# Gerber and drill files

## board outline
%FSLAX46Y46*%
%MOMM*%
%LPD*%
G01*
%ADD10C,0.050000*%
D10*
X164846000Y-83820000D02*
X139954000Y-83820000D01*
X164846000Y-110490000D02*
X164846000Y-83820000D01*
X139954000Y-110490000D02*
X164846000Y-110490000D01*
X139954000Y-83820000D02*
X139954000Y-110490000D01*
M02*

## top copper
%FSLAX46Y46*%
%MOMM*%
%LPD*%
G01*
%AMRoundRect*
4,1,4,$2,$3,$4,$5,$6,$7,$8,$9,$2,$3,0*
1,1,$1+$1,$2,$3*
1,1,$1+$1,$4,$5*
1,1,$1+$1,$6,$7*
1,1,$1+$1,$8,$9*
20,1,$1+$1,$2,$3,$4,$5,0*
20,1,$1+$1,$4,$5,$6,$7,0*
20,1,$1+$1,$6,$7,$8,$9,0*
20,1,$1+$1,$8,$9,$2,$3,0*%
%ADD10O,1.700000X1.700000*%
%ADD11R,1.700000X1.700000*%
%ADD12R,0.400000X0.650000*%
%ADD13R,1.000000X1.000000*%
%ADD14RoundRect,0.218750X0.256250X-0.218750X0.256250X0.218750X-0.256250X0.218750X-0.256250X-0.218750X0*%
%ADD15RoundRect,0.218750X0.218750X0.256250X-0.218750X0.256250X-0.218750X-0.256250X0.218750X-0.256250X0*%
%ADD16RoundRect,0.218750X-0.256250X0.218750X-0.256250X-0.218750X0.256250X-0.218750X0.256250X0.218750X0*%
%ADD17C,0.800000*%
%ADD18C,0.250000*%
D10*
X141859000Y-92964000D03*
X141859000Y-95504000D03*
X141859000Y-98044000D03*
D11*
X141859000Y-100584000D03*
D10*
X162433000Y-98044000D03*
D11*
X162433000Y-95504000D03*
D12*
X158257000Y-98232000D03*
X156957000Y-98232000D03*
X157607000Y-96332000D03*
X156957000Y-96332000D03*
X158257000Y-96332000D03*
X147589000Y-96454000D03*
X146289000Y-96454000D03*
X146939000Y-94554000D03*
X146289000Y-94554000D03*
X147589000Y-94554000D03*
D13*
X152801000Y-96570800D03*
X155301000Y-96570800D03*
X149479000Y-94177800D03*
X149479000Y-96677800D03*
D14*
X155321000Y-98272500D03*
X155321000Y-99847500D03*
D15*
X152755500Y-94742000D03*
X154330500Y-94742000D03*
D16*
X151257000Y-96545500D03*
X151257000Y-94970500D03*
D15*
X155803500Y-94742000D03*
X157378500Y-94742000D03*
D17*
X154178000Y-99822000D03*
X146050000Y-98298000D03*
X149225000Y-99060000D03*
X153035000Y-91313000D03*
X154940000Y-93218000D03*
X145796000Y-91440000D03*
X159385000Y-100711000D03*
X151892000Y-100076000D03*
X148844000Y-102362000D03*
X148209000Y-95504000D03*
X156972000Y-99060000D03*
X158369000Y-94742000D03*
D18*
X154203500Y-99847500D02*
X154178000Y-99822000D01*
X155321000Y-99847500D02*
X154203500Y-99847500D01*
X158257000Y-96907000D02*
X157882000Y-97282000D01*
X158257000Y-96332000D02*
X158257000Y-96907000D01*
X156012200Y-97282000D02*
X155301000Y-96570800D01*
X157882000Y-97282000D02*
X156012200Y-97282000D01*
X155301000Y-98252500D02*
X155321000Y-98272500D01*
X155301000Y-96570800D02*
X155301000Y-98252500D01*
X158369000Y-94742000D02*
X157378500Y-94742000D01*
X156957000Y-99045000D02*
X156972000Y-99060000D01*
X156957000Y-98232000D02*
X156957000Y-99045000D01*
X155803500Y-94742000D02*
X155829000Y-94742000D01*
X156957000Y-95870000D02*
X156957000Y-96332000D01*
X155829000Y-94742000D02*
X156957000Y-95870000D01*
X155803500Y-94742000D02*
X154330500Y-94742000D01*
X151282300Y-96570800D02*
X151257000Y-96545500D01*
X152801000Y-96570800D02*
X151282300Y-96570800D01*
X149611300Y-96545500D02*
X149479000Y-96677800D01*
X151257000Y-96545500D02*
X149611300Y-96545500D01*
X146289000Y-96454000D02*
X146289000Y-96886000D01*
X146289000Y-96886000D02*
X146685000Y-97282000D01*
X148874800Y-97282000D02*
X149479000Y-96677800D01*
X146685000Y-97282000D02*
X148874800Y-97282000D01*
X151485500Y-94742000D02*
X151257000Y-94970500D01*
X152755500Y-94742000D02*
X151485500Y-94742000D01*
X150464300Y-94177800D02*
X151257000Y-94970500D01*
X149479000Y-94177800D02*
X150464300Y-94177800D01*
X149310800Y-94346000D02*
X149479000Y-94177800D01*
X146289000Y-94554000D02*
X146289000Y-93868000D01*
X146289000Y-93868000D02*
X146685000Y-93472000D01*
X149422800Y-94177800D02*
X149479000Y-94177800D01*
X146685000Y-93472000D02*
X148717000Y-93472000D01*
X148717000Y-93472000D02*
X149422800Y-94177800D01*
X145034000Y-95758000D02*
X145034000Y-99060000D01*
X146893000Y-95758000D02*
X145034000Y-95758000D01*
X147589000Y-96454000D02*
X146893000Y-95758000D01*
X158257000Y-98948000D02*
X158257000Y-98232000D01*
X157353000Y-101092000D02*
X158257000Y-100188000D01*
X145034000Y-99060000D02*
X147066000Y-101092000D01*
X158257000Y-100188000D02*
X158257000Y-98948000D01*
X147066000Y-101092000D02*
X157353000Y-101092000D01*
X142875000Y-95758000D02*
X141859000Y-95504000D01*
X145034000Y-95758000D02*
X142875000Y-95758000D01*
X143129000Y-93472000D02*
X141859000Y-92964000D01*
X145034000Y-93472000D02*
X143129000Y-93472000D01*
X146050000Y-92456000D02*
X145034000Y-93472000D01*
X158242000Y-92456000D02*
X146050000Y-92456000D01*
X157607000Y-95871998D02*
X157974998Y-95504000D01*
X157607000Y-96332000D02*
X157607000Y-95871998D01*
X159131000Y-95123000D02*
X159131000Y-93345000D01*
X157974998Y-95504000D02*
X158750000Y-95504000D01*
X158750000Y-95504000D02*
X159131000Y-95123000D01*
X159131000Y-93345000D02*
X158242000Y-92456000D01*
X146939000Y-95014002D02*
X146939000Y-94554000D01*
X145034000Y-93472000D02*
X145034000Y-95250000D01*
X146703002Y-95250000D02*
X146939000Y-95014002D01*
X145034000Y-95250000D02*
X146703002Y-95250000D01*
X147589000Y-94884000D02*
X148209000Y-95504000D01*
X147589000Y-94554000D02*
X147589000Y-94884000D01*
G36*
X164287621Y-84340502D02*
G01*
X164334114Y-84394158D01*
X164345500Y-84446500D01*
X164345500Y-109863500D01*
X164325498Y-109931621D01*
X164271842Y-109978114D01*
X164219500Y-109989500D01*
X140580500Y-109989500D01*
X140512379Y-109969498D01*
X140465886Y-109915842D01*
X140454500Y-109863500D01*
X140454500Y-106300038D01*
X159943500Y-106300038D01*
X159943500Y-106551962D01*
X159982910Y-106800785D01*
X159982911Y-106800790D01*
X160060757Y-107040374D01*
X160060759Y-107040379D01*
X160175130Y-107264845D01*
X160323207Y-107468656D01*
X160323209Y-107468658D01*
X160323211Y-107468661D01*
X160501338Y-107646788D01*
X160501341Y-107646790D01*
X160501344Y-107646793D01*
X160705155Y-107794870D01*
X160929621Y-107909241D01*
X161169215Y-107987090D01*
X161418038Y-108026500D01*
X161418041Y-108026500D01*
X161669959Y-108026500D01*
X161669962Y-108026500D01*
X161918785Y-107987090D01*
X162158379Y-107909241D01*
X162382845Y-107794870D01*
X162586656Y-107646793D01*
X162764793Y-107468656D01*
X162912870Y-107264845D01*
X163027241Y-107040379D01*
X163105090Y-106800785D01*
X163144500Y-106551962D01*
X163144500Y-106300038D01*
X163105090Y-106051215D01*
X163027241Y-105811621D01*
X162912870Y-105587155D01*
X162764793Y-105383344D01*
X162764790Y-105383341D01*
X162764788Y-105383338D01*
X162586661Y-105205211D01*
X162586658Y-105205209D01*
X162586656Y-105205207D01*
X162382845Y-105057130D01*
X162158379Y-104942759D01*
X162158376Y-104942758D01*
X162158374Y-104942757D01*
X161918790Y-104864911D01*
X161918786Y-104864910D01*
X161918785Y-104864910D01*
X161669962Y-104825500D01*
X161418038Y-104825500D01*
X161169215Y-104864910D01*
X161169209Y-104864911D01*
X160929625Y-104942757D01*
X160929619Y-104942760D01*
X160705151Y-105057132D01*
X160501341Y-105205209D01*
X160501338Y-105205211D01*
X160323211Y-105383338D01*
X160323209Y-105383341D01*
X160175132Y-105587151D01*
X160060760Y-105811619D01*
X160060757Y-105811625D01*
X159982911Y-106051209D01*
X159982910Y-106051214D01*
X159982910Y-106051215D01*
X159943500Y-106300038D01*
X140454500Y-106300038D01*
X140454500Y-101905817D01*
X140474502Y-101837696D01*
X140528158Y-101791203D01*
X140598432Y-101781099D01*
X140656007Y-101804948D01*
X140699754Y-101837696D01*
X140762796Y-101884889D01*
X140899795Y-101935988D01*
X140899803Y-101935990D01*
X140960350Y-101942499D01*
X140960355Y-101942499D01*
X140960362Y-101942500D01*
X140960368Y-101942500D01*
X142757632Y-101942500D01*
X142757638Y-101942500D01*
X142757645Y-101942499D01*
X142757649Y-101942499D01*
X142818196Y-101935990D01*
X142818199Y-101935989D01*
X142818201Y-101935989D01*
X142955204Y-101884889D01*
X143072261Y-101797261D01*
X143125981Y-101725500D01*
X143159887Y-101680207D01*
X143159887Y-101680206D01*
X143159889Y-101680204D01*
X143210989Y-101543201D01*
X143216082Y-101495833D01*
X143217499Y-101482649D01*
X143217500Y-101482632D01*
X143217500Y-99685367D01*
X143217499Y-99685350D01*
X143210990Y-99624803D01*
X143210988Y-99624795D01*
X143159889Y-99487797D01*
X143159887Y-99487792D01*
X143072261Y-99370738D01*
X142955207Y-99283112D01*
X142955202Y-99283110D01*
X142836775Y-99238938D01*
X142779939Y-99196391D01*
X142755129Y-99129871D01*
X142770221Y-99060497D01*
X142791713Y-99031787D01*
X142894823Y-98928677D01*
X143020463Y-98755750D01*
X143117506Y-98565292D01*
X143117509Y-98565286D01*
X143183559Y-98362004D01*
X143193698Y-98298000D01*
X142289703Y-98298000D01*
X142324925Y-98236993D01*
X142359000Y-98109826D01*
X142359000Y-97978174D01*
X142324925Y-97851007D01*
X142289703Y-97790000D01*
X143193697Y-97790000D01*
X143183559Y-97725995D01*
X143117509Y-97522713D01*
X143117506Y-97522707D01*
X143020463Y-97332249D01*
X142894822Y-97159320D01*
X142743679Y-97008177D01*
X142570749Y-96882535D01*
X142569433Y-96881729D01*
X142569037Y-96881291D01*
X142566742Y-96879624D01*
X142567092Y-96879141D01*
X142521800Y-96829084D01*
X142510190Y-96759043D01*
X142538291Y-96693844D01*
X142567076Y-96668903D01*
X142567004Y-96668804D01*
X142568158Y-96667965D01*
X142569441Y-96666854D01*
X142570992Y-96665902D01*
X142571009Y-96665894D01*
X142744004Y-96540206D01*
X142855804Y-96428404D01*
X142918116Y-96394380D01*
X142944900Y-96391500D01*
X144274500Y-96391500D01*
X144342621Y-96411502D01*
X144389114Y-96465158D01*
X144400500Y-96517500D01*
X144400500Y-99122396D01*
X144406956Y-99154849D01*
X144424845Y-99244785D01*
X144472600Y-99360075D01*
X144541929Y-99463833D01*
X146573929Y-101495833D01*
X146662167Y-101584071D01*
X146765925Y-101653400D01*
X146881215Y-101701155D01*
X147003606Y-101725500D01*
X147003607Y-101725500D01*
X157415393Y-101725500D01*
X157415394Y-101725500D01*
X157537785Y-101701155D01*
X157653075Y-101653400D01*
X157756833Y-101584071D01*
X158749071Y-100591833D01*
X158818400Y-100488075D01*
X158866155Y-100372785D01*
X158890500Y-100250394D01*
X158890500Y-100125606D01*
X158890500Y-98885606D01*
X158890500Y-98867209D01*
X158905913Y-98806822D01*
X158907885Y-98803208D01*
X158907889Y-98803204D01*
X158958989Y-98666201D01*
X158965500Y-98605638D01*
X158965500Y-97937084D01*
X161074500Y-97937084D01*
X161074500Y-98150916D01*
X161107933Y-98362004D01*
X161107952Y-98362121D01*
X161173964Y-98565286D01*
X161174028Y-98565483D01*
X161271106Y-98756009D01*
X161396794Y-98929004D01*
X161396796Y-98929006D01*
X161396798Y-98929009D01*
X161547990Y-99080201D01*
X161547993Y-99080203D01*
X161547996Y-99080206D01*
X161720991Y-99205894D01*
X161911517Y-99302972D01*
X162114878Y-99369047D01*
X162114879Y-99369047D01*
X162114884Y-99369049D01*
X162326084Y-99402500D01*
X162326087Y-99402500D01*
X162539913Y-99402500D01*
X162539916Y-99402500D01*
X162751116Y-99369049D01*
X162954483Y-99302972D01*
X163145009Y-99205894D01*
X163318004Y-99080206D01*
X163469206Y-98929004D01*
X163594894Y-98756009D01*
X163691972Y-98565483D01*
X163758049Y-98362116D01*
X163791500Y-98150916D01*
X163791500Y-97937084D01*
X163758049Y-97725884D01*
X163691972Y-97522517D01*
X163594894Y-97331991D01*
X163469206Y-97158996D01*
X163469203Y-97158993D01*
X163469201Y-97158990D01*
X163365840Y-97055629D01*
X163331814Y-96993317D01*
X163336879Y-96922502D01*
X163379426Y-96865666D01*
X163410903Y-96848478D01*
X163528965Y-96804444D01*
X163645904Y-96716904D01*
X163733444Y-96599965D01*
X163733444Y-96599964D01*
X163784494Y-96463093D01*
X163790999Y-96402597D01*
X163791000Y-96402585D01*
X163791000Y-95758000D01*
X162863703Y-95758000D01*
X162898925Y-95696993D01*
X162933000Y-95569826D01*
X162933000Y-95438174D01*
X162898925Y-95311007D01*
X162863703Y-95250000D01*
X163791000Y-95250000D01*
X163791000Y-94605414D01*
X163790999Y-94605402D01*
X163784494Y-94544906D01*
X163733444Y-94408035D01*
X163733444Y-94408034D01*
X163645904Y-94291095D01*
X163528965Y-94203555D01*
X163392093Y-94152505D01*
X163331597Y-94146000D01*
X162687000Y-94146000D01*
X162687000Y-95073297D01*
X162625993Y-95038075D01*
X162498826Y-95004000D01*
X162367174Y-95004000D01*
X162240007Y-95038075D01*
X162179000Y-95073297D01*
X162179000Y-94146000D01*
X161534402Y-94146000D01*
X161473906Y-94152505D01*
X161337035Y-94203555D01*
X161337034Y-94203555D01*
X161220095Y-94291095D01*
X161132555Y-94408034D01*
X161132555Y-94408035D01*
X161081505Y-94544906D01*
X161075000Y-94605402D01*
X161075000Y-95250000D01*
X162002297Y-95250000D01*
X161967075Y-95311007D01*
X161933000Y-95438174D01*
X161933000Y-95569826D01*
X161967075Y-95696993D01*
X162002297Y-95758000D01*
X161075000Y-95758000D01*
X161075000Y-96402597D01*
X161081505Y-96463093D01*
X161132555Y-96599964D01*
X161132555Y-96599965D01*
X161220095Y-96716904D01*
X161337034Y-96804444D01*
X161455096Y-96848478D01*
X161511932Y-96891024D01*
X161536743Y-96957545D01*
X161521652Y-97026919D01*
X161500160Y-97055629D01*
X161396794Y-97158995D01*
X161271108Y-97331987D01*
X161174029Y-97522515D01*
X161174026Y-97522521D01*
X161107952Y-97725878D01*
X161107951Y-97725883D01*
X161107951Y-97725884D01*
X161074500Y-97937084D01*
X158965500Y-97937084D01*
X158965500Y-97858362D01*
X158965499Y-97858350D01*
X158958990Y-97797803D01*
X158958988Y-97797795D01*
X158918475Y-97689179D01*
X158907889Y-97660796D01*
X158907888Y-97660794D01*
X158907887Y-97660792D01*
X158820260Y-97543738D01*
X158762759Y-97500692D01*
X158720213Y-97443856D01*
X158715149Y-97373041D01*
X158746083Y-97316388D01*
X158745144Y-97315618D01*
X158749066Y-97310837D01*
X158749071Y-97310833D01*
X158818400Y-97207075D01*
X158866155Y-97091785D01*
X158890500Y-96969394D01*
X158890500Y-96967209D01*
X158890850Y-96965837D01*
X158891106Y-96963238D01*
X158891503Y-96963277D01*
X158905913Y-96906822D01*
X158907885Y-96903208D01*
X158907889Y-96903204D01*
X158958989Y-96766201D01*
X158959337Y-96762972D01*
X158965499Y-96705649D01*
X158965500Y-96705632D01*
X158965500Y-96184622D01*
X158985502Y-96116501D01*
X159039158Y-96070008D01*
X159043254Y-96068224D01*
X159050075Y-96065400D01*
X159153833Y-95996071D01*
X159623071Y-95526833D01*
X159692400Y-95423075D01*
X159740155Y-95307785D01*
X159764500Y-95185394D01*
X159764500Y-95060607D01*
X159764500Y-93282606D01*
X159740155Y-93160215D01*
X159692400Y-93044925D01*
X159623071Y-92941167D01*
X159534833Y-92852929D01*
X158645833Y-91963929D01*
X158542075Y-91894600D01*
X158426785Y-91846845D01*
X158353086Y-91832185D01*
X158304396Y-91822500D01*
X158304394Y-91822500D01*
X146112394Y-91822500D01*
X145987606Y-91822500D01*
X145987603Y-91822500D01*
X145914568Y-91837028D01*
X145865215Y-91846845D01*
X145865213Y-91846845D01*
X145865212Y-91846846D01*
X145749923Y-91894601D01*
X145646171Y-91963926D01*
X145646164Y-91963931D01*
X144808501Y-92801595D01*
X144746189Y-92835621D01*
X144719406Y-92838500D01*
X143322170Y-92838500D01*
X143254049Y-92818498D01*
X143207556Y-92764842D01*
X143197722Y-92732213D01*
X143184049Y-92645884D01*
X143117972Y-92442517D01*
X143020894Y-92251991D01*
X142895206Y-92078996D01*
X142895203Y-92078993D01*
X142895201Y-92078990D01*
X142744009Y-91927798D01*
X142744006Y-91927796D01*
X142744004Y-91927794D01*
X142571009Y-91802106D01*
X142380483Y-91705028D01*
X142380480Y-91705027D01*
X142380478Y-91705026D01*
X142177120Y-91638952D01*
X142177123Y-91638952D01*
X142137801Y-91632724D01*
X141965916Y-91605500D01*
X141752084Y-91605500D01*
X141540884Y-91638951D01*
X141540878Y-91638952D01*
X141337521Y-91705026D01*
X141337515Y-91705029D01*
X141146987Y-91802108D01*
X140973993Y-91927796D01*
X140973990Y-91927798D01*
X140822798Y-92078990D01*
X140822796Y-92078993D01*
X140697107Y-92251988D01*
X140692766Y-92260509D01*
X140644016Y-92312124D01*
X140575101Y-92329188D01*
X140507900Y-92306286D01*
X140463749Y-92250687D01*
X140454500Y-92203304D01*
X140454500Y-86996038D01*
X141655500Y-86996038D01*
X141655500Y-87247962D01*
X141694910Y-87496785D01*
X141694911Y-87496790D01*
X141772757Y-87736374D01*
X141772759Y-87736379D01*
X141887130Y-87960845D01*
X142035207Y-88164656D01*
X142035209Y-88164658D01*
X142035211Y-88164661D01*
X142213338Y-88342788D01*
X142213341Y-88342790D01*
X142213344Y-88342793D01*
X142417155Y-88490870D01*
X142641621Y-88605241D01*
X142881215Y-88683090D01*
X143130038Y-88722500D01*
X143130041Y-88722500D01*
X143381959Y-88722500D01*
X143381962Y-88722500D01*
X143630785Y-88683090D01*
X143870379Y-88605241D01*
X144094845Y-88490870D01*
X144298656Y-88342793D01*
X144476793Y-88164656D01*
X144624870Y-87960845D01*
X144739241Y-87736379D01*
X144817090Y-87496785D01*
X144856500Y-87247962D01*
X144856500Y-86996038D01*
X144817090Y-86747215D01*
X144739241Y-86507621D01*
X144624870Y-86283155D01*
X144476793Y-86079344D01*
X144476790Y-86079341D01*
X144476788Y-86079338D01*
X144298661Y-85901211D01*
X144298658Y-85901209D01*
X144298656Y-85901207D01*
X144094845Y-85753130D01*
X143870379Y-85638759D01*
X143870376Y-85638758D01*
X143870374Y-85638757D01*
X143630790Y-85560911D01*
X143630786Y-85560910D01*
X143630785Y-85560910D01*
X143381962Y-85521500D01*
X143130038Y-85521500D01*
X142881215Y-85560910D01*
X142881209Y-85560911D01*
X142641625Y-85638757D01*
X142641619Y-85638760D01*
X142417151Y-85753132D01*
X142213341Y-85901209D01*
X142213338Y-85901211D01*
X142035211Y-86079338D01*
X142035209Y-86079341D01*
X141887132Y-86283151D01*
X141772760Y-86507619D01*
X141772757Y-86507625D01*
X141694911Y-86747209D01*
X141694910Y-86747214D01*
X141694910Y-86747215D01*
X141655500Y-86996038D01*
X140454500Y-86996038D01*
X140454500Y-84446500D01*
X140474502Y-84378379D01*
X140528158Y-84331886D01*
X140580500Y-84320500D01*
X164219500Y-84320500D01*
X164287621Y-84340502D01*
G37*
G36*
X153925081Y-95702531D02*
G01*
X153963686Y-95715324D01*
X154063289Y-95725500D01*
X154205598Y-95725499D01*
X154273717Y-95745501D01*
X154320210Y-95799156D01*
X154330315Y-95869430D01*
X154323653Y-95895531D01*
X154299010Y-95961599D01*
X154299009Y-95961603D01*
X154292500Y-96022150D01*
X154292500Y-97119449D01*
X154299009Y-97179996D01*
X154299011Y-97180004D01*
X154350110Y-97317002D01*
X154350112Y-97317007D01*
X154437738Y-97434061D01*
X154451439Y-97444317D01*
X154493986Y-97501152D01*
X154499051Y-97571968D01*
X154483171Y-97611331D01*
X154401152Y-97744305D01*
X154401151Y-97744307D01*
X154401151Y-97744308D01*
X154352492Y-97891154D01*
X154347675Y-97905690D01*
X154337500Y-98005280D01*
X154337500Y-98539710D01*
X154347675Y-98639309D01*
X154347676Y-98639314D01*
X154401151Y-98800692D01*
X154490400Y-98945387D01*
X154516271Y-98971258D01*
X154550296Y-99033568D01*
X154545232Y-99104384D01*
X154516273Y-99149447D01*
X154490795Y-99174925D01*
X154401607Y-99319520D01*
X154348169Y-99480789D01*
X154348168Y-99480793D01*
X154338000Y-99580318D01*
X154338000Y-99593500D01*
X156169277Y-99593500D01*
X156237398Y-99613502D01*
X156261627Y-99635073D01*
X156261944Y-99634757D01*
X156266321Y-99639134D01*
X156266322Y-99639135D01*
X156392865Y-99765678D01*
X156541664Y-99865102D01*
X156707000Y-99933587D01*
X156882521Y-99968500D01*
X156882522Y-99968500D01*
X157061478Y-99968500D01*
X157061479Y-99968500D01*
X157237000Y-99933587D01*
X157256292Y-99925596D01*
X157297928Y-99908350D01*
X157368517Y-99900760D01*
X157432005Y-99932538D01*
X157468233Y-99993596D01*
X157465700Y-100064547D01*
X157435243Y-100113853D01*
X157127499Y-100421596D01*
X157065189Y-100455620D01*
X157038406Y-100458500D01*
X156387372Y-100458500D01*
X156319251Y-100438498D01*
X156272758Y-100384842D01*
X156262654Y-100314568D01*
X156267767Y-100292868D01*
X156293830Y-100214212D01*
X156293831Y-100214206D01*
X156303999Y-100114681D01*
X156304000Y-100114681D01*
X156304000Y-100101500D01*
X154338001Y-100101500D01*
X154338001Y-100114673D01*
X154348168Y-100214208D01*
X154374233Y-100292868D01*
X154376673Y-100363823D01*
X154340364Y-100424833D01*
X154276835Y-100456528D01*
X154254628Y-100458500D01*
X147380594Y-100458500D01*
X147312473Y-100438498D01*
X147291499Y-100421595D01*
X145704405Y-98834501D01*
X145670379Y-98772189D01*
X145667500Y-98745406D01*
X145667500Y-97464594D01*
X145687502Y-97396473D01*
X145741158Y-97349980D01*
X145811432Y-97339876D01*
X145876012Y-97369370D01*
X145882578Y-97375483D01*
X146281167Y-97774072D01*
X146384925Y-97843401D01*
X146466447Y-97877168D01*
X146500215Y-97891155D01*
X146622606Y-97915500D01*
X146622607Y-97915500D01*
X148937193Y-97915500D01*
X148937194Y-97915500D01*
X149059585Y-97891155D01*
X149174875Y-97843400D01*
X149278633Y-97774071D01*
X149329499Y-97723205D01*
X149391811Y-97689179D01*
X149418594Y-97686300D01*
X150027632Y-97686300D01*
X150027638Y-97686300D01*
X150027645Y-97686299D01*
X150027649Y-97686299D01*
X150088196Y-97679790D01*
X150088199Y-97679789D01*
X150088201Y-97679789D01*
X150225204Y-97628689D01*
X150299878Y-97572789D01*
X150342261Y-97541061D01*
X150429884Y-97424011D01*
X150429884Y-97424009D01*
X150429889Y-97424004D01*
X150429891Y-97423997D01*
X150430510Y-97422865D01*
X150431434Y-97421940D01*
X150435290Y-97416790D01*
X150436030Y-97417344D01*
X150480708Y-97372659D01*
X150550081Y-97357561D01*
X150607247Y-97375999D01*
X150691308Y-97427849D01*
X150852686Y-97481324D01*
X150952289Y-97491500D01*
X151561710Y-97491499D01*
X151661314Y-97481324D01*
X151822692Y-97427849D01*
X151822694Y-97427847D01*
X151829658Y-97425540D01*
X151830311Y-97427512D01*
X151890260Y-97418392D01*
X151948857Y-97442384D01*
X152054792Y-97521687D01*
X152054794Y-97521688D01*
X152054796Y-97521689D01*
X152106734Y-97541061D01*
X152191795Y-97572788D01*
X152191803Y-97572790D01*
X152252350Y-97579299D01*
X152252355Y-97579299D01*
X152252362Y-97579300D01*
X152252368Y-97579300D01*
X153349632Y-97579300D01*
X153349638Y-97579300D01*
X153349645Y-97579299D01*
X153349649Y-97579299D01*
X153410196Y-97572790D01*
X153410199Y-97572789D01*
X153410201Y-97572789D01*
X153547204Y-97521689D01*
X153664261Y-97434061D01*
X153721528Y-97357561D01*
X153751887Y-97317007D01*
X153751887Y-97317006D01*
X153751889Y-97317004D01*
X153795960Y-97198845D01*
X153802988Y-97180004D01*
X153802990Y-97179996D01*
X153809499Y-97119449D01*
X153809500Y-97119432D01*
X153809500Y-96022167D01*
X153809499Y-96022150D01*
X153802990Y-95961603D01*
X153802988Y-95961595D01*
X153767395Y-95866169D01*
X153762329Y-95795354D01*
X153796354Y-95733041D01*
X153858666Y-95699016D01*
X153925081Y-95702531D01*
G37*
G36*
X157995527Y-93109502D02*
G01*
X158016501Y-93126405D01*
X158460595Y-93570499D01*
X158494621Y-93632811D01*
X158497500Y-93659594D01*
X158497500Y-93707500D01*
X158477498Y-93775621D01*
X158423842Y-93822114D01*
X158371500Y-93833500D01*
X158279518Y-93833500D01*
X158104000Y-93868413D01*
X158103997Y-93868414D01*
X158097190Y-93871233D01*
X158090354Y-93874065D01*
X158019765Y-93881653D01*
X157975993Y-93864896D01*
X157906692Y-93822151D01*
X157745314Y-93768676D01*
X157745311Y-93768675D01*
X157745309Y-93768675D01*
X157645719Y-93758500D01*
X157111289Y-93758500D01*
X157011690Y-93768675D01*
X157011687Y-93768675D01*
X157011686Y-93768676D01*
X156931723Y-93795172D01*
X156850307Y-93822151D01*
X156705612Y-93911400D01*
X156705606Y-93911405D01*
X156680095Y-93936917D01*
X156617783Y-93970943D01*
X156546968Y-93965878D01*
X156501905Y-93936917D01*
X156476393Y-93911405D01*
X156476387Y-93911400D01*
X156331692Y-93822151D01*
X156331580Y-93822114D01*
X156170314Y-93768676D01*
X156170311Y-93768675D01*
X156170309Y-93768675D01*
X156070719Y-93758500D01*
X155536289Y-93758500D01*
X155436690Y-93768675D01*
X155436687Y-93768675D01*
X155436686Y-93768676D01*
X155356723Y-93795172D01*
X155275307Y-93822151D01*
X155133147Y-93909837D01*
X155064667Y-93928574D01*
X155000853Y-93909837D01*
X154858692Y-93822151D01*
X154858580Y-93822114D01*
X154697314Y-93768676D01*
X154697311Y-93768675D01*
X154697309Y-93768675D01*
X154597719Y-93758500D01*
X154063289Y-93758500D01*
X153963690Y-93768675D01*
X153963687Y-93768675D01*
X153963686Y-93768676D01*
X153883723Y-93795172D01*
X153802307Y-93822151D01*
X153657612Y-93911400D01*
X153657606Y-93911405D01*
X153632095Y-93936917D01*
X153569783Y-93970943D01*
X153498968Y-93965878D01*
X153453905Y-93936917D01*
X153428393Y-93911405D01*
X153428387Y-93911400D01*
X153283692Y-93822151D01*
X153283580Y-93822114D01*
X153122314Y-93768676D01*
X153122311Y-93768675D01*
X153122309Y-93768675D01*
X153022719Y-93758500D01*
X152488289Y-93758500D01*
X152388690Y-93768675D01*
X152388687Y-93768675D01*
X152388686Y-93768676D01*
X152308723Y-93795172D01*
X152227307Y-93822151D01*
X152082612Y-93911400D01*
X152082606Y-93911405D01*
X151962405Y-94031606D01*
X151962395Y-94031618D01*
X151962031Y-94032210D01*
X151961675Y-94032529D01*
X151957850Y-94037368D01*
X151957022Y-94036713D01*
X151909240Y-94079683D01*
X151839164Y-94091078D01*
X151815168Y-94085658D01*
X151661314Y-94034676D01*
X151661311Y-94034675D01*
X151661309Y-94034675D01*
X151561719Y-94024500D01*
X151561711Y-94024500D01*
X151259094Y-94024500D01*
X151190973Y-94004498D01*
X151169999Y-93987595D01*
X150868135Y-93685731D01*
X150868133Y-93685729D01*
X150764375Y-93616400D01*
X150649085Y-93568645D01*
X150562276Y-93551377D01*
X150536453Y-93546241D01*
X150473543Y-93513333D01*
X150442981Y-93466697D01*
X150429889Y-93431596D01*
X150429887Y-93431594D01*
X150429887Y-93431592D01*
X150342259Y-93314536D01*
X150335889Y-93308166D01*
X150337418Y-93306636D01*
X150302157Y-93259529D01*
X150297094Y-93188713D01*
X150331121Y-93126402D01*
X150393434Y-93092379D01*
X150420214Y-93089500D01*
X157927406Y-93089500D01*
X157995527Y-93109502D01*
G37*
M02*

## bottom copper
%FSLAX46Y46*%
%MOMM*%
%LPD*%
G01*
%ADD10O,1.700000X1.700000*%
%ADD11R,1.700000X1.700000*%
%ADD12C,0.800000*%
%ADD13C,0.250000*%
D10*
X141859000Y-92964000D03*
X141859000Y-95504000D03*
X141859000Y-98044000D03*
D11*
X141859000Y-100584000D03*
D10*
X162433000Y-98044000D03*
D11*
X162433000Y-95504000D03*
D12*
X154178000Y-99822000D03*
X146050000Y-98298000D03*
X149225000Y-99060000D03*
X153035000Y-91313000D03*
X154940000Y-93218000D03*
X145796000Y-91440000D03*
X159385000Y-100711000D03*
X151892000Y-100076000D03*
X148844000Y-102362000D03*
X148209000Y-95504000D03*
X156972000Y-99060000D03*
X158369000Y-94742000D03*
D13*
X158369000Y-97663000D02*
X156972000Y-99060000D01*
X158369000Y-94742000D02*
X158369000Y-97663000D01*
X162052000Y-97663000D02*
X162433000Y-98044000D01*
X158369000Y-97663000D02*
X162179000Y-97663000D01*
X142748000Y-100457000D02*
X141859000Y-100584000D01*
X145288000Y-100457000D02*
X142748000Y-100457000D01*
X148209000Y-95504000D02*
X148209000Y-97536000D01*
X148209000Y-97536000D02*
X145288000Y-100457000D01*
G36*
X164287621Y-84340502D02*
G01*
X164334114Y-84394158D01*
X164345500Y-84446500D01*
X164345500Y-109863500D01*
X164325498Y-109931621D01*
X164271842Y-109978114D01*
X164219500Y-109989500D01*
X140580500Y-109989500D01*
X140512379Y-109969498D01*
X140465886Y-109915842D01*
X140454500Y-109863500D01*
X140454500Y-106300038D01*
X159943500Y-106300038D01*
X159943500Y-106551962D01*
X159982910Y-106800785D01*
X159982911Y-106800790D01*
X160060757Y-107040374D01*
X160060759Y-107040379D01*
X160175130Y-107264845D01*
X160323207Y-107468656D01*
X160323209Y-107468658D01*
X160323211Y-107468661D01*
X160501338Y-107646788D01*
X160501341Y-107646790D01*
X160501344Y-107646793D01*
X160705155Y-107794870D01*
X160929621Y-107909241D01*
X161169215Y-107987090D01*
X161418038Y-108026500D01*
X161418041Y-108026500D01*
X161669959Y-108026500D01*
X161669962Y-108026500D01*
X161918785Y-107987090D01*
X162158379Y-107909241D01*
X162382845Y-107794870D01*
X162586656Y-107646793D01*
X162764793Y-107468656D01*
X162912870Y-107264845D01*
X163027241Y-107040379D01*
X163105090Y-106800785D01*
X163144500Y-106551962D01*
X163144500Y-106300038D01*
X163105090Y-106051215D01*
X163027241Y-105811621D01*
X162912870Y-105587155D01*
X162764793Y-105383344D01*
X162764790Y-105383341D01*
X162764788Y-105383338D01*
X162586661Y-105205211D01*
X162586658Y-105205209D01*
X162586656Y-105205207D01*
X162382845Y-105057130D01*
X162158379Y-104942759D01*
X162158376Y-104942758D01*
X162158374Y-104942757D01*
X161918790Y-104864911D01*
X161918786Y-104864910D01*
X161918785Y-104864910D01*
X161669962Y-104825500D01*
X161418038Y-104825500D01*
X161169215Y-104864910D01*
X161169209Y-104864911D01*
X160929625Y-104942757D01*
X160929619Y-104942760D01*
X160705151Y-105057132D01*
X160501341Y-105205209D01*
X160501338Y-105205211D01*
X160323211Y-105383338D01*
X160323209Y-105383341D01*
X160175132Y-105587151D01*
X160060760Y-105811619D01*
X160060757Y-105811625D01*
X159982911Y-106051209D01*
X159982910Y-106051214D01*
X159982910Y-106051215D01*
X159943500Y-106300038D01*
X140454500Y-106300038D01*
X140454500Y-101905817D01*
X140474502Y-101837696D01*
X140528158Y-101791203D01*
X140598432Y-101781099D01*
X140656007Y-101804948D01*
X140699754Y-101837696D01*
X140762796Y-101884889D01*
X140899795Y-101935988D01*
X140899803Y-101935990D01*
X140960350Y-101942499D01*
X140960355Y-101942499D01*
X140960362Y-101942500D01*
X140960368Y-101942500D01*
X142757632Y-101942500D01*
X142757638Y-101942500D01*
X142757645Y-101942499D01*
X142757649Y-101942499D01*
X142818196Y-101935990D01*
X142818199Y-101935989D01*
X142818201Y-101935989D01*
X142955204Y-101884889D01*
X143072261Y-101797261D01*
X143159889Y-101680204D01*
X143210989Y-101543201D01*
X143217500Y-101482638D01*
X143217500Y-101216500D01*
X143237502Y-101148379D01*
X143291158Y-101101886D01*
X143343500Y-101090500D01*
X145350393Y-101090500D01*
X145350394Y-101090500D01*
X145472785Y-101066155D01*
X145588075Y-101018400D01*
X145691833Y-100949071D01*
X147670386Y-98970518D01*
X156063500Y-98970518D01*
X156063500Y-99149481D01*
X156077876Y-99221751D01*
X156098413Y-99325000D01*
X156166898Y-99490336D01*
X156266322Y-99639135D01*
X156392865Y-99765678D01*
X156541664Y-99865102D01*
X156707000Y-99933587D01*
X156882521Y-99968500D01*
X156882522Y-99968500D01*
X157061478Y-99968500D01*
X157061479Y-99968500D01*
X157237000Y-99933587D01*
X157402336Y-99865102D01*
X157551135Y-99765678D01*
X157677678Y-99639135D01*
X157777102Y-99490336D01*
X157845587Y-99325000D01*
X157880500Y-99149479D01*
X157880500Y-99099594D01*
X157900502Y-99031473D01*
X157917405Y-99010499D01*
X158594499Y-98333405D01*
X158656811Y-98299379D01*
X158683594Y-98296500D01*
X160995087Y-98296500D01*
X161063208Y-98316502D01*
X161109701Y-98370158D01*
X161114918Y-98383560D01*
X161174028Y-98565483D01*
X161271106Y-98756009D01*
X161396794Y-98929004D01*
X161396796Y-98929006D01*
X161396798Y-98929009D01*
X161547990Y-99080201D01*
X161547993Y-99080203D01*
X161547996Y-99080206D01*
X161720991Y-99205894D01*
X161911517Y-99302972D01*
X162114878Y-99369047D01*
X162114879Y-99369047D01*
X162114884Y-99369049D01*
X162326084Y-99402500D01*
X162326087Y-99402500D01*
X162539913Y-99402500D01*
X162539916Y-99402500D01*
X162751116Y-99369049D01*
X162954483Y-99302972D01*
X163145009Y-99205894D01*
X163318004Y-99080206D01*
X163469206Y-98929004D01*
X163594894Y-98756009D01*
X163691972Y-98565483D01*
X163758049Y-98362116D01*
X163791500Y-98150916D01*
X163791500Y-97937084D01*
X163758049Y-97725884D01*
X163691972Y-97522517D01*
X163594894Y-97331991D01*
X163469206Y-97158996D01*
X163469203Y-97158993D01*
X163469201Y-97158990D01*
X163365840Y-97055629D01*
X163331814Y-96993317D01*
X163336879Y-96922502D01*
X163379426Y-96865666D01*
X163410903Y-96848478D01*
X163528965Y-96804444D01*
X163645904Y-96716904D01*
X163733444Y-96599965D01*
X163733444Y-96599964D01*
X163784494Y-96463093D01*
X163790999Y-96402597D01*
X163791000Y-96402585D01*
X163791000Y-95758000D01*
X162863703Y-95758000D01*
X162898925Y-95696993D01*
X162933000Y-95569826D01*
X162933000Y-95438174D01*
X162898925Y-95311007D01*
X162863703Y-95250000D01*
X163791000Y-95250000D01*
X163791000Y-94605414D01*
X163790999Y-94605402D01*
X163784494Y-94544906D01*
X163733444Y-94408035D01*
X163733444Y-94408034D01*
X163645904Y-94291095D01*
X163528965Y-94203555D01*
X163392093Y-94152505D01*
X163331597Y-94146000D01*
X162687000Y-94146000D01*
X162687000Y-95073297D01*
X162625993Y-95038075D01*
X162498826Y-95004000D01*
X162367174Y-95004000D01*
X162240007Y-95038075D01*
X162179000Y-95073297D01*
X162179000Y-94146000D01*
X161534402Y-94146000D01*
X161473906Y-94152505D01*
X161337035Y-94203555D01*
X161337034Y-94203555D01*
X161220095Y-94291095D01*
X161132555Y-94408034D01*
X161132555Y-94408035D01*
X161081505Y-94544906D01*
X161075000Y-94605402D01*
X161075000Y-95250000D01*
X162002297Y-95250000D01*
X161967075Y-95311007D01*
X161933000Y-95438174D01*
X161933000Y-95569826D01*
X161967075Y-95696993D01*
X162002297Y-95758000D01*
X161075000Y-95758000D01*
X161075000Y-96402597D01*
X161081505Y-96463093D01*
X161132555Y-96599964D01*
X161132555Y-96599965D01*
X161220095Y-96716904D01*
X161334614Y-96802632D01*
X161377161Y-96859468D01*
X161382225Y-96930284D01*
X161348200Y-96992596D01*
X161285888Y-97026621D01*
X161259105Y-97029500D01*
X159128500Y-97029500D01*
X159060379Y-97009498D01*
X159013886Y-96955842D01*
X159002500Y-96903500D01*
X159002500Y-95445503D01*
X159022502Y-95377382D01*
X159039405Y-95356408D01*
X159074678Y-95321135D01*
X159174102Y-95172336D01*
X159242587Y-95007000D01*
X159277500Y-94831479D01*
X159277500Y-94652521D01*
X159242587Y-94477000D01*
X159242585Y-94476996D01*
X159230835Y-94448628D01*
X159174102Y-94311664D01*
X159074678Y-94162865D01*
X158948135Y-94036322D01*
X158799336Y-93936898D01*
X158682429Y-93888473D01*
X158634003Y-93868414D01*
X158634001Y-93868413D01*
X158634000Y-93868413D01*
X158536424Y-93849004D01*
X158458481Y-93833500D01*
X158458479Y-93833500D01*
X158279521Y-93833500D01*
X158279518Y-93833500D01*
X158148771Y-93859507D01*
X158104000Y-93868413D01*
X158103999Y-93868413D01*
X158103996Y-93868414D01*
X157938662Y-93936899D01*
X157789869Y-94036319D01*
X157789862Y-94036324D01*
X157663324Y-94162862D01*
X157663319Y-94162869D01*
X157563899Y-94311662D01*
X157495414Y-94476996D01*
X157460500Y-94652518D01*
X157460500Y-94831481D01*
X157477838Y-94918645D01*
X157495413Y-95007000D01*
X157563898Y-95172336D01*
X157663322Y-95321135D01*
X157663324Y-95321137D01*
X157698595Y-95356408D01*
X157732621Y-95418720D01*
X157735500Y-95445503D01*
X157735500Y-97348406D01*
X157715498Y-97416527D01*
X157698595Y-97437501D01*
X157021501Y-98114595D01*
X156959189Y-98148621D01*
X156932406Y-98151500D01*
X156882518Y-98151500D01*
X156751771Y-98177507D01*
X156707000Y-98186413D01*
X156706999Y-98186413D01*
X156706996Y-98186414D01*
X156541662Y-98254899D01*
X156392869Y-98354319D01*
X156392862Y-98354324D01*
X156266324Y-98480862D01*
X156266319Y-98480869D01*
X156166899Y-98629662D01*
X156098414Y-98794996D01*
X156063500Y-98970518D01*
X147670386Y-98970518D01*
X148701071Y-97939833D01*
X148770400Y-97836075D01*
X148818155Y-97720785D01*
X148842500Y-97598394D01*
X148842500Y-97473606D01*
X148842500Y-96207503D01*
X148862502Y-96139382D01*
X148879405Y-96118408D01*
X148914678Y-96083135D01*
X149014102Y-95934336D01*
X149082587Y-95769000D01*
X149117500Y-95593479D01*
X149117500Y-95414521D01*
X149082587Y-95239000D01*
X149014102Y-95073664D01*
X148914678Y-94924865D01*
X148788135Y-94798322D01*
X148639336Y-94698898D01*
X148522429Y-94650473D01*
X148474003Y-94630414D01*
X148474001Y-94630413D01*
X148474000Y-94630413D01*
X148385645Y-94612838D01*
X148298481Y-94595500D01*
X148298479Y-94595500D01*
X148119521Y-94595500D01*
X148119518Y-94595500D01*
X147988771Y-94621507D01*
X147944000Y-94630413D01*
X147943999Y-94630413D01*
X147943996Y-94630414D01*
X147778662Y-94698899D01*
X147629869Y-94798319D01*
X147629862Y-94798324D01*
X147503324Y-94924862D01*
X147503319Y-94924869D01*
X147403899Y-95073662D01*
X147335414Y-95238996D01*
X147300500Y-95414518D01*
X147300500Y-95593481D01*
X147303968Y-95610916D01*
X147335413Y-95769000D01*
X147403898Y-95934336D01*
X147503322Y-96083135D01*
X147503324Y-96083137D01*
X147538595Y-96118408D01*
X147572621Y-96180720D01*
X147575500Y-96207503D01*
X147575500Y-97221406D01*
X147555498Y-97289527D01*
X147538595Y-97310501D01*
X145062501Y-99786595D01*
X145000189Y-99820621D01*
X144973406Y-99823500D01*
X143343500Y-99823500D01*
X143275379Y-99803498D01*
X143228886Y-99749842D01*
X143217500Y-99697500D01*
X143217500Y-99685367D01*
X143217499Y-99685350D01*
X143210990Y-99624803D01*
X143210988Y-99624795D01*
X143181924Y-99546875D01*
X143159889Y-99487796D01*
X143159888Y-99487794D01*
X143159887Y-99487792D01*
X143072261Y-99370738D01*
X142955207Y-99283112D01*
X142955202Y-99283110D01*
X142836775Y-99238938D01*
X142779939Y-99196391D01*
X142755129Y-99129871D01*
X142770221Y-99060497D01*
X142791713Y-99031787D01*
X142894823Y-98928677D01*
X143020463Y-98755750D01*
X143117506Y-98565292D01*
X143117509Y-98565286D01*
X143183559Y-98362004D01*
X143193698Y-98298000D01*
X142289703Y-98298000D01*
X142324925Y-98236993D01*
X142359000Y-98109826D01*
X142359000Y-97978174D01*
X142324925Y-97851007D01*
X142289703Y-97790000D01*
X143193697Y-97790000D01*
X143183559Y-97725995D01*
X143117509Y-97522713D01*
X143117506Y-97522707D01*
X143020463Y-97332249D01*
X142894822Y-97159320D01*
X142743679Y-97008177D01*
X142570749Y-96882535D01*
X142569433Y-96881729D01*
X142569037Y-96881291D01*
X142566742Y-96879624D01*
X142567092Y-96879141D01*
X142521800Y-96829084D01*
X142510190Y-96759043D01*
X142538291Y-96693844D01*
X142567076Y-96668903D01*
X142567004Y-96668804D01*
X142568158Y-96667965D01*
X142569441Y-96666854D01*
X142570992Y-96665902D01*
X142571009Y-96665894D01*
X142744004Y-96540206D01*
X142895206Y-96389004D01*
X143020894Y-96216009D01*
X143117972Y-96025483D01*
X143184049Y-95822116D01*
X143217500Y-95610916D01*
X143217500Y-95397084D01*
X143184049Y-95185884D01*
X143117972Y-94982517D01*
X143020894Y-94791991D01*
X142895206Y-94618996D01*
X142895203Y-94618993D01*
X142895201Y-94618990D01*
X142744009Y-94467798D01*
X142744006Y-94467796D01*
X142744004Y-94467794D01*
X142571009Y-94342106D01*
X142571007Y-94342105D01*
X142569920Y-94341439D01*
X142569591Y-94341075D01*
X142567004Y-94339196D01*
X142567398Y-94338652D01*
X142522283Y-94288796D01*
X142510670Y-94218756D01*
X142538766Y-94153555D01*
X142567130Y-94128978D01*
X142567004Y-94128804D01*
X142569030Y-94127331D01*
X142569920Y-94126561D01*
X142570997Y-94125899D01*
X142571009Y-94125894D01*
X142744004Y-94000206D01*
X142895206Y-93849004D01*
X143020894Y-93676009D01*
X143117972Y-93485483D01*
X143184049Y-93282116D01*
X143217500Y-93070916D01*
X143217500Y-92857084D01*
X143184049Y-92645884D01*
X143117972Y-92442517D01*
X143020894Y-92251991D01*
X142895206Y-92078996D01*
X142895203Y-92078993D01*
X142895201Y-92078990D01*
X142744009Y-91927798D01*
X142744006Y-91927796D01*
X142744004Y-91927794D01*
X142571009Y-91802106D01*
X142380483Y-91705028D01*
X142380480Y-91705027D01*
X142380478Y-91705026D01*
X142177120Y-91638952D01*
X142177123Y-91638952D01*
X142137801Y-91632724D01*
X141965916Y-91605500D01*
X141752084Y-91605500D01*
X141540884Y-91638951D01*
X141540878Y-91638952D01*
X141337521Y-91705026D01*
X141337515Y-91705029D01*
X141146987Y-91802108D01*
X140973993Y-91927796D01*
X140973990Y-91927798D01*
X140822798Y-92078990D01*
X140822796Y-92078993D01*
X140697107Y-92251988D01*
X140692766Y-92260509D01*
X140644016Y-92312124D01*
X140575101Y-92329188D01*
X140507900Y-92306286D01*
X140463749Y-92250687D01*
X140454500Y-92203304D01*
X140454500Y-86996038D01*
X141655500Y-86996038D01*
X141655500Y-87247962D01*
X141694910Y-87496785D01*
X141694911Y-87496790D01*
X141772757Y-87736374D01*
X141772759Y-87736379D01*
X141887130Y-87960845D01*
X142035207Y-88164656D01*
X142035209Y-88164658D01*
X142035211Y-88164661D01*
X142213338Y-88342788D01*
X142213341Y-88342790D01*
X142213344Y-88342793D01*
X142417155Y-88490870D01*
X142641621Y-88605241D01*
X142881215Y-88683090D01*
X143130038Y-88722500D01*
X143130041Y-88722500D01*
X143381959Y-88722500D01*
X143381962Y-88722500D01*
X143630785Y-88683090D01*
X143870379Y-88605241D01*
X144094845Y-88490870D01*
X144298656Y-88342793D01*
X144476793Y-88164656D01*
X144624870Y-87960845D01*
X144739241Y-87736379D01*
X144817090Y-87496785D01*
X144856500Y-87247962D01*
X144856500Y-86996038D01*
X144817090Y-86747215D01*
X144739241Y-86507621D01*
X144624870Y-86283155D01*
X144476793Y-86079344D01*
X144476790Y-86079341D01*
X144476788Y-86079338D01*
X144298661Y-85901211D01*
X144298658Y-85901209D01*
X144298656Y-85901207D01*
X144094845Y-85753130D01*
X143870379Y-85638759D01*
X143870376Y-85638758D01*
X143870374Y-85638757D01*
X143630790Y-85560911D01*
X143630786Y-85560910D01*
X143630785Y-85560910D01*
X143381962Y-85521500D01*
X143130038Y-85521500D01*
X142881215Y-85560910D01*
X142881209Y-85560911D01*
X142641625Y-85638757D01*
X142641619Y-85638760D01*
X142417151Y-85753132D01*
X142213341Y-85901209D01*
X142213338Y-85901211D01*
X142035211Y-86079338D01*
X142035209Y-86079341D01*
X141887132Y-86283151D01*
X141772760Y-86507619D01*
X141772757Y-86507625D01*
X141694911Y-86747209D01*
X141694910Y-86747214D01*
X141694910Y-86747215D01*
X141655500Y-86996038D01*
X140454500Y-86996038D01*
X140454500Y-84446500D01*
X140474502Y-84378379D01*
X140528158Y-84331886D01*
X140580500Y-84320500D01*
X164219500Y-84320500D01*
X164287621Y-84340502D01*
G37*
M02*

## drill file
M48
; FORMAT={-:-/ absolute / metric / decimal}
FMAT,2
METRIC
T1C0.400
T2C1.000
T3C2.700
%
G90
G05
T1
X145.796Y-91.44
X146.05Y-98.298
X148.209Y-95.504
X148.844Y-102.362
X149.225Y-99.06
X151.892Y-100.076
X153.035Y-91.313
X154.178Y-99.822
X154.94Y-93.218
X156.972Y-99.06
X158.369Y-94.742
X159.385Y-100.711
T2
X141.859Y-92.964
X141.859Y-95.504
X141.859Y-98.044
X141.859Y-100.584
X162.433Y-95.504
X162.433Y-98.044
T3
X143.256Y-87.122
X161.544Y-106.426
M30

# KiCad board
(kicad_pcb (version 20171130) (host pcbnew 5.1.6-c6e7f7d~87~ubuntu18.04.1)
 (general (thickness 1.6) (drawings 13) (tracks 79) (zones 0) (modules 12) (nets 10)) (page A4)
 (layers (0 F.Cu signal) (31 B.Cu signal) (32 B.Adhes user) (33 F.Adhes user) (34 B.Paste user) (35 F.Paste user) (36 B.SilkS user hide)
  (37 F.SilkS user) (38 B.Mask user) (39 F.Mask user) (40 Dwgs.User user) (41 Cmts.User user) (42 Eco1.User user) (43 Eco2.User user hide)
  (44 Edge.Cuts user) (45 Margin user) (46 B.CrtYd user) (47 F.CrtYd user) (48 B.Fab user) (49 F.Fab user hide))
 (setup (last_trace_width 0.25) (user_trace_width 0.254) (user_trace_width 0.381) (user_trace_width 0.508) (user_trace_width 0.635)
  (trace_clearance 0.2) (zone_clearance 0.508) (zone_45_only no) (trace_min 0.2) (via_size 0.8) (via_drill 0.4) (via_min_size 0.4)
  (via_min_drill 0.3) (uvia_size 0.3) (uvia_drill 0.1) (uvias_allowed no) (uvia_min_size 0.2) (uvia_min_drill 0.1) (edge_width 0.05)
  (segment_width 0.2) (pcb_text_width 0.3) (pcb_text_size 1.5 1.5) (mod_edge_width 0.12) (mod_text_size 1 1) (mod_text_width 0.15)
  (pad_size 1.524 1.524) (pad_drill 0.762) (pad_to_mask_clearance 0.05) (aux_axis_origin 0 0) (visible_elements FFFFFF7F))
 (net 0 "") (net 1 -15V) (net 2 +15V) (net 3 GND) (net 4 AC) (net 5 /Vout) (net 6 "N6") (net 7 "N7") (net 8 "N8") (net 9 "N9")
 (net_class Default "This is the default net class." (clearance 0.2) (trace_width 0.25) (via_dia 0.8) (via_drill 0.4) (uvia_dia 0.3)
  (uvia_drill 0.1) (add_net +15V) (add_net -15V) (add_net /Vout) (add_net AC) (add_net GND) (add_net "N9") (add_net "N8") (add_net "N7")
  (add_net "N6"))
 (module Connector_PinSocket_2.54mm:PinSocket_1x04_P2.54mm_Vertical (layer F.Cu) (at 141.859 100.584 180)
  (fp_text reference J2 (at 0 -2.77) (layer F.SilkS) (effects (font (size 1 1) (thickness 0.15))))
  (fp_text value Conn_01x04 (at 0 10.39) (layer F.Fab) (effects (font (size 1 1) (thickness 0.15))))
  (pad 4 thru_hole oval (at 0 7.62 180) (size 1.7 1.7) (drill 1) (layers *.Cu *.Mask) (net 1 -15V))
  (pad 3 thru_hole oval (at 0 5.08 180) (size 1.7 1.7) (drill 1) (layers *.Cu *.Mask) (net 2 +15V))
  (pad 2 thru_hole oval (at 0 2.54 180) (size 1.7 1.7) (drill 1) (layers *.Cu *.Mask) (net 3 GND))
  (pad 1 thru_hole rect (at 0 0 180) (size 1.7 1.7) (drill 1) (layers *.Cu *.Mask) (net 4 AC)))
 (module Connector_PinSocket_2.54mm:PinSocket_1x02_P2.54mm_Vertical (layer F.Cu) (at 162.433 95.504)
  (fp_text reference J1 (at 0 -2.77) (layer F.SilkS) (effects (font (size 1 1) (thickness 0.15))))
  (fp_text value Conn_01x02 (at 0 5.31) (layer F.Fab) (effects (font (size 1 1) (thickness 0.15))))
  (pad 2 thru_hole oval (at 0 2.54) (size 1.7 1.7) (drill 1) (layers *.Cu *.Mask) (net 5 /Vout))
  (pad 1 thru_hole rect (at 0 0) (size 1.7 1.7) (drill 1) (layers *.Cu *.Mask) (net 3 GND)))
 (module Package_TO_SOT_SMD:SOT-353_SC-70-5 (layer F.Cu) (at 157.607 97.282 270)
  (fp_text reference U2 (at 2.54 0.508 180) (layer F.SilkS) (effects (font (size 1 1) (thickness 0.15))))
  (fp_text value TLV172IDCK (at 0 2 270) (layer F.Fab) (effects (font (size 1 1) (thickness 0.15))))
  (pad 5 smd rect (at 0.95 -0.65 270) (size 0.65 0.4) (layers F.Cu F.Paste F.Mask) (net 2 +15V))
  (pad 4 smd rect (at 0.95 0.65 270) (size 0.65 0.4) (layers F.Cu F.Paste F.Mask) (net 5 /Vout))
  (pad 2 smd rect (at -0.95 0 270) (size 0.65 0.4) (layers F.Cu F.Paste F.Mask) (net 1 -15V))
  (pad 3 smd rect (at -0.95 0.65 270) (size 0.65 0.4) (layers F.Cu F.Paste F.Mask) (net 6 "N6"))
  (pad 1 smd rect (at -0.95 -0.65 270) (size 0.65 0.4) (layers F.Cu F.Paste F.Mask) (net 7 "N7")))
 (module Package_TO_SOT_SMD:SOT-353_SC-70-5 (layer F.Cu) (at 146.939 95.504 270)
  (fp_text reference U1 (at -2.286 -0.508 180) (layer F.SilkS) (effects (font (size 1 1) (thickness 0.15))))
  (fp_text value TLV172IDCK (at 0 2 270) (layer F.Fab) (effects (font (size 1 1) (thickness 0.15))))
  (pad 5 smd rect (at 0.95 -0.65 270) (size 0.65 0.4) (layers F.Cu F.Paste F.Mask) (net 2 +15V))
  (pad 4 smd rect (at 0.95 0.65 270) (size 0.65 0.4) (layers F.Cu F.Paste F.Mask) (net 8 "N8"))
  (pad 2 smd rect (at -0.95 0 270) (size 0.65 0.4) (layers F.Cu F.Paste F.Mask) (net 1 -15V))
  (pad 3 smd rect (at -0.95 0.65 270) (size 0.65 0.4) (layers F.Cu F.Paste F.Mask) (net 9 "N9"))
  (pad 1 smd rect (at -0.95 -0.65 270) (size 0.65 0.4) (layers F.Cu F.Paste F.Mask) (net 4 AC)))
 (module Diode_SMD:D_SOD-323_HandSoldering (layer F.Cu) (at 154.051 96.5708 180)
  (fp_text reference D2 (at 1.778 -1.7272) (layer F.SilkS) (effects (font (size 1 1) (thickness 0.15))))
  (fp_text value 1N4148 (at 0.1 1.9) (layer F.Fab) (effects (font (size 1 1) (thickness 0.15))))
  (pad 2 smd rect (at 1.25 0 180) (size 1 1) (layers F.Cu F.Paste F.Mask) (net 8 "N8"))
  (pad 1 smd rect (at -1.25 0 180) (size 1 1) (layers F.Cu F.Paste F.Mask) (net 7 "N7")))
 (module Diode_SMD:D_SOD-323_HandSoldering (layer F.Cu) (at 149.479 95.4278 90)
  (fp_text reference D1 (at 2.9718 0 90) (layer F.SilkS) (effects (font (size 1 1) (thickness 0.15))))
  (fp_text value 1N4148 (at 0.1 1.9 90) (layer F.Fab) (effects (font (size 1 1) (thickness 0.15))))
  (pad 2 smd rect (at 1.25 0 90) (size 1 1) (layers F.Cu F.Paste F.Mask) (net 9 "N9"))
  (pad 1 smd rect (at -1.25 0 90) (size 1 1) (layers F.Cu F.Paste F.Mask) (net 8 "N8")))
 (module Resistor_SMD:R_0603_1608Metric (layer F.Cu) (at 155.321 99.06 90)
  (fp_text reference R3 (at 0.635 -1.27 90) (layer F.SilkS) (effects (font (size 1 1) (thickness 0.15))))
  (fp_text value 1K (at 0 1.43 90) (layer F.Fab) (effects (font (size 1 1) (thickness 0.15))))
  (pad 2 smd roundrect (at 0.7875 0 90) (size 0.875 0.95) (layers F.Cu F.Paste F.Mask) (roundrect_rratio 0.25) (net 7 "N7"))
  (pad 1 smd roundrect (at -0.7875 0 90) (size 0.875 0.95) (layers F.Cu F.Paste F.Mask) (roundrect_rratio 0.25) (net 3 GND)))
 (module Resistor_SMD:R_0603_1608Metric (layer F.Cu) (at 153.543 94.742 180)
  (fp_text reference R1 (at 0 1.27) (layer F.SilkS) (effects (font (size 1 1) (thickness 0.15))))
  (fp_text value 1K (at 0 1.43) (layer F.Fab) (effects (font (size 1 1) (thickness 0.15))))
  (pad 2 smd roundrect (at 0.7875 0 180) (size 0.875 0.95) (layers F.Cu F.Paste F.Mask) (roundrect_rratio 0.25) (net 9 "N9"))
  (pad 1 smd roundrect (at -0.7875 0 180) (size 0.875 0.95) (layers F.Cu F.Paste F.Mask) (roundrect_rratio 0.25) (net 6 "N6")))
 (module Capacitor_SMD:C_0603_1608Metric (layer F.Cu) (at 151.257 95.758 270)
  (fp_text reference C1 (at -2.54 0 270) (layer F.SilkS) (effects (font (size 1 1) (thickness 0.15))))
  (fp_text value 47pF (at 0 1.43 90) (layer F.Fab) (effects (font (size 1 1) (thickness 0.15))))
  (pad 2 smd roundrect (at 0.7875 0 270) (size 0.875 0.95) (layers F.Cu F.Paste F.Mask) (roundrect_rratio 0.25) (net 8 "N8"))
  (pad 1 smd roundrect (at -0.7875 0 270) (size 0.875 0.95) (layers F.Cu F.Paste F.Mask) (roundrect_rratio 0.25) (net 9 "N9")))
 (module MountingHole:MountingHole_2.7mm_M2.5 (layer F.Cu) (at 161.544 106.426)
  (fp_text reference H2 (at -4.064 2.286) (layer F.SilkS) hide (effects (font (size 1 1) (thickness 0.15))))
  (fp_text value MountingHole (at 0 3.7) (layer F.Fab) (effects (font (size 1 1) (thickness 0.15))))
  (pad 1 np_thru_hole circle (at 0 0) (size 2.7 2.7) (drill 2.7) (layers *.Cu *.Mask)))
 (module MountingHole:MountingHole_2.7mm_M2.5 (layer F.Cu) (at 143.256 87.122)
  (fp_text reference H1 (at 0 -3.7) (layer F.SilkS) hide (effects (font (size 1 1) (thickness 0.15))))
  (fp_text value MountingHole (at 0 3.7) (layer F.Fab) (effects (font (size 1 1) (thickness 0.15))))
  (pad 1 np_thru_hole circle (at 0 0) (size 2.7 2.7) (drill 2.7) (layers *.Cu *.Mask)))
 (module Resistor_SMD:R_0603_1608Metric (layer F.Cu) (at 156.591 94.742 180)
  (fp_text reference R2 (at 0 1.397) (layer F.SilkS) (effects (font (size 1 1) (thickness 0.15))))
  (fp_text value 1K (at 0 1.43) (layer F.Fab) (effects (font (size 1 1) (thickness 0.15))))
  (pad 2 smd roundrect (at 0.7875 0 180) (size 0.875 0.95) (layers F.Cu F.Paste F.Mask) (roundrect_rratio 0.25) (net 6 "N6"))
  (pad 1 smd roundrect (at -0.7875 0 180) (size 0.875 0.95) (layers F.Cu F.Paste F.Mask) (roundrect_rratio 0.25) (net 5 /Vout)))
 (gr_line (start 164.846 83.82) (end 139.954 83.82) (layer Edge.Cuts) (width 0.05))
 (gr_line (start 164.846 110.49) (end 164.846 83.82) (layer Edge.Cuts) (width 0.05))
 (gr_line (start 139.954 110.49) (end 164.846 110.49) (layer Edge.Cuts) (width 0.05))
 (gr_line (start 139.954 83.82) (end 139.954 110.49) (layer Edge.Cuts) (width 0.05))
 (via (at 154.178 99.822) (size 0.8) (drill 0.4) (layers F.Cu B.Cu) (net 3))
 (segment (start 154.2035 99.8475) (end 154.178 99.822) (width 0.25) (layer F.Cu) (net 3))
 (segment (start 155.321 99.8475) (end 154.2035 99.8475) (width 0.25) (layer F.Cu) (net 3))
 (via (at 146.05 98.298) (size 0.8) (drill 0.4) (layers F.Cu B.Cu) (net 3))
 (via (at 149.225 99.06) (size 0.8) (drill 0.4) (layers F.Cu B.Cu) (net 3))
 (via (at 153.035 91.313) (size 0.8) (drill 0.4) (layers F.Cu B.Cu) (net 3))
 (via (at 154.94 93.218) (size 0.8) (drill 0.4) (layers F.Cu B.Cu) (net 3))
 (via (at 145.796 91.44) (size 0.8) (drill 0.4) (layers F.Cu B.Cu) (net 3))
 (via (at 159.385 100.711) (size 0.8) (drill 0.4) (layers F.Cu B.Cu) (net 3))
 (via (at 151.892 100.076) (size 0.8) (drill 0.4) (layers F.Cu B.Cu) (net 3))
 (via (at 148.844 102.362) (size 0.8) (drill 0.4) (layers F.Cu B.Cu) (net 3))
 (via (at 148.209 95.504) (size 0.8) (drill 0.4) (layers F.Cu B.Cu) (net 4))
 (via (at 156.972 99.06) (size 0.8) (drill 0.4) (layers F.Cu B.Cu) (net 5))
 (via (at 158.369 94.742) (size 0.8) (drill 0.4) (layers F.Cu B.Cu) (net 5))
 (segment (start 158.257 96.907) (end 157.882 97.282) (width 0.25) (layer F.Cu) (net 7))
 (segment (start 158.257 96.332) (end 158.257 96.907) (width 0.25) (layer F.Cu) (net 7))
 (segment (start 156.0122 97.282) (end 155.301 96.5708) (width 0.25) (layer F.Cu) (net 7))
 (segment (start 157.882 97.282) (end 156.0122 97.282) (width 0.25) (layer F.Cu) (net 7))
 (segment (start 155.301 98.2525) (end 155.321 98.2725) (width 0.25) (layer F.Cu) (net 7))
 (segment (start 155.301 96.5708) (end 155.301 98.2525) (width 0.25) (layer F.Cu) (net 7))
 (segment (start 158.369 94.742) (end 157.3785 94.742) (width 0.25) (layer F.Cu) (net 5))
 (segment (start 158.369 97.663) (end 156.972 99.06) (width 0.25) (layer B.Cu) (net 5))
 (segment (start 158.369 94.742) (end 158.369 97.663) (width 0.25) (layer B.Cu) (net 5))
 (segment (start 156.957 99.045) (end 156.972 99.06) (width 0.25) (layer F.Cu) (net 5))
 (segment (start 156.957 98.232) (end 156.957 99.045) (width 0.25) (layer F.Cu) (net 5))
 (segment (start 162.052 97.663) (end 162.433 98.044) (width 0.25) (layer B.Cu) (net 5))
 (segment (start 158.369 97.663) (end 162.179 97.663) (width 0.25) (layer B.Cu) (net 5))
 (segment (start 155.8035 94.742) (end 155.829 94.742) (width 0.25) (layer F.Cu) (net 6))
 (segment (start 156.957 95.87) (end 156.957 96.332) (width 0.25) (layer F.Cu) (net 6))
 (segment (start 155.829 94.742) (end 156.957 95.87) (width 0.25) (layer F.Cu) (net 6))
 (segment (start 155.8035 94.742) (end 154.3305 94.742) (width 0.25) (layer F.Cu) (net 6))
 (segment (start 151.2823 96.5708) (end 151.257 96.5455) (width 0.25) (layer F.Cu) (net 8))
 (segment (start 152.801 96.5708) (end 151.2823 96.5708) (width 0.25) (layer F.Cu) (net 8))
 (segment (start 149.6113 96.5455) (end 149.479 96.6778) (width 0.25) (layer F.Cu) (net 8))
 (segment (start 151.257 96.5455) (end 149.6113 96.5455) (width 0.25) (layer F.Cu) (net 8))
 (segment (start 146.289 96.454) (end 146.289 96.886) (width 0.25) (layer F.Cu) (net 8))
 (segment (start 146.289 96.886) (end 146.685 97.282) (width 0.25) (layer F.Cu) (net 8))
 (segment (start 148.8748 97.282) (end 149.479 96.6778) (width 0.25) (layer F.Cu) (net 8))
 (segment (start 146.685 97.282) (end 148.8748 97.282) (width 0.25) (layer F.Cu) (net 8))
 (segment (start 151.4855 94.742) (end 151.257 94.9705) (width 0.25) (layer F.Cu) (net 9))
 (segment (start 152.7555 94.742) (end 151.4855 94.742) (width 0.25) (layer F.Cu) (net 9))
 (segment (start 150.4643 94.1778) (end 151.257 94.9705) (width 0.25) (layer F.Cu) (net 9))
 (segment (start 149.479 94.1778) (end 150.4643 94.1778) (width 0.25) (layer F.Cu) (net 9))
 (segment (start 149.3108 94.346) (end 149.479 94.1778) (width 0.25) (layer F.Cu) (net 9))
 (segment (start 146.289 94.554) (end 146.289 93.868) (width 0.25) (layer F.Cu) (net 9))
 (segment (start 146.289 93.868) (end 146.685 93.472) (width 0.25) (layer F.Cu) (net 9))
 (segment (start 149.4228 94.1778) (end 149.479 94.1778) (width 0.25) (layer F.Cu) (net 9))
 (segment (start 146.685 93.472) (end 148.717 93.472) (width 0.25) (layer F.Cu) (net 9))
 (segment (start 148.717 93.472) (end 149.4228 94.1778) (width 0.25) (layer F.Cu) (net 9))
 (segment (start 145.034 95.758) (end 145.034 99.06) (width 0.25) (layer F.Cu) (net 2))
 (segment (start 146.893 95.758) (end 145.034 95.758) (width 0.25) (layer F.Cu) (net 2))
 (segment (start 147.589 96.454) (end 146.893 95.758) (width 0.25) (layer F.Cu) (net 2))
 (segment (start 158.257 98.948) (end 158.257 98.232) (width 0.25) (layer F.Cu) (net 2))
 (segment (start 157.353 101.092) (end 158.257 100.188) (width 0.25) (layer F.Cu) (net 2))
 (segment (start 145.034 99.06) (end 147.066 101.092) (width 0.25) (layer F.Cu) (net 2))
 (segment (start 158.257 100.188) (end 158.257 98.948) (width 0.25) (layer F.Cu) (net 2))
 (segment (start 147.066 101.092) (end 157.353 101.092) (width 0.25) (layer F.Cu) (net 2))
 (segment (start 142.875 95.758) (end 141.859 95.504) (width 0.25) (layer F.Cu) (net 2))
 (segment (start 145.034 95.758) (end 142.875 95.758) (width 0.25) (layer F.Cu) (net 2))
 (segment (start 143.129 93.472) (end 141.859 92.964) (width 0.25) (layer F.Cu) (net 1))
 (segment (start 145.034 93.472) (end 143.129 93.472) (width 0.25) (layer F.Cu) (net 1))
 (segment (start 146.05 92.456) (end 145.034 93.472) (width 0.25) (layer F.Cu) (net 1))
 (segment (start 158.242 92.456) (end 146.05 92.456) (width 0.25) (layer F.Cu) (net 1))
 (segment (start 157.607 95.871998) (end 157.974998 95.504) (width 0.25) (layer F.Cu) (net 1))
 (segment (start 157.607 96.332) (end 157.607 95.871998) (width 0.25) (layer F.Cu) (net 1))
 (segment (start 159.131 95.123) (end 159.131 93.345) (width 0.25) (layer F.Cu) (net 1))
 (segment (start 157.974998 95.504) (end 158.75 95.504) (width 0.25) (layer F.Cu) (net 1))
 (segment (start 158.75 95.504) (end 159.131 95.123) (width 0.25) (layer F.Cu) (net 1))
 (segment (start 159.131 93.345) (end 158.242 92.456) (width 0.25) (layer F.Cu) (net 1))
 (segment (start 146.939 95.014002) (end 146.939 94.554) (width 0.25) (layer F.Cu) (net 1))
 (segment (start 145.034 93.472) (end 145.034 95.25) (width 0.25) (layer F.Cu) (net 1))
 (segment (start 146.703002 95.25) (end 146.939 95.014002) (width 0.25) (layer F.Cu) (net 1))
 (segment (start 145.034 95.25) (end 146.703002 95.25) (width 0.25) (layer F.Cu) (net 1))
 (segment (start 147.589 94.884) (end 148.209 95.504) (width 0.25) (layer F.Cu) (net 4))
 (segment (start 147.589 94.554) (end 147.589 94.884) (width 0.25) (layer F.Cu) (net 4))
 (segment (start 142.748 100.457) (end 141.859 100.584) (width 0.25) (layer B.Cu) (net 4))
 (segment (start 145.288 100.457) (end 142.748 100.457) (width 0.25) (layer B.Cu) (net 4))
 (segment (start 148.209 95.504) (end 148.209 97.536) (width 0.25) (layer B.Cu) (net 4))
 (segment (start 148.209 97.536) (end 145.288 100.457) (width 0.25) (layer B.Cu) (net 4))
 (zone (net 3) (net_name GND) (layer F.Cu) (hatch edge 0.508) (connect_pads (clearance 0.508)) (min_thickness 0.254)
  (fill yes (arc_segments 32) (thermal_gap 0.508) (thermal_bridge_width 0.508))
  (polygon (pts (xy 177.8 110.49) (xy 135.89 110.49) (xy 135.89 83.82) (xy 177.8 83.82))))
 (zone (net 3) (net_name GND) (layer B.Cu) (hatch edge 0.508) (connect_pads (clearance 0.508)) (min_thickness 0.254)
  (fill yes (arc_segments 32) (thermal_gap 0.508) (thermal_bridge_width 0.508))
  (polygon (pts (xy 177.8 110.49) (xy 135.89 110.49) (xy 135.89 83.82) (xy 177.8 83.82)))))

